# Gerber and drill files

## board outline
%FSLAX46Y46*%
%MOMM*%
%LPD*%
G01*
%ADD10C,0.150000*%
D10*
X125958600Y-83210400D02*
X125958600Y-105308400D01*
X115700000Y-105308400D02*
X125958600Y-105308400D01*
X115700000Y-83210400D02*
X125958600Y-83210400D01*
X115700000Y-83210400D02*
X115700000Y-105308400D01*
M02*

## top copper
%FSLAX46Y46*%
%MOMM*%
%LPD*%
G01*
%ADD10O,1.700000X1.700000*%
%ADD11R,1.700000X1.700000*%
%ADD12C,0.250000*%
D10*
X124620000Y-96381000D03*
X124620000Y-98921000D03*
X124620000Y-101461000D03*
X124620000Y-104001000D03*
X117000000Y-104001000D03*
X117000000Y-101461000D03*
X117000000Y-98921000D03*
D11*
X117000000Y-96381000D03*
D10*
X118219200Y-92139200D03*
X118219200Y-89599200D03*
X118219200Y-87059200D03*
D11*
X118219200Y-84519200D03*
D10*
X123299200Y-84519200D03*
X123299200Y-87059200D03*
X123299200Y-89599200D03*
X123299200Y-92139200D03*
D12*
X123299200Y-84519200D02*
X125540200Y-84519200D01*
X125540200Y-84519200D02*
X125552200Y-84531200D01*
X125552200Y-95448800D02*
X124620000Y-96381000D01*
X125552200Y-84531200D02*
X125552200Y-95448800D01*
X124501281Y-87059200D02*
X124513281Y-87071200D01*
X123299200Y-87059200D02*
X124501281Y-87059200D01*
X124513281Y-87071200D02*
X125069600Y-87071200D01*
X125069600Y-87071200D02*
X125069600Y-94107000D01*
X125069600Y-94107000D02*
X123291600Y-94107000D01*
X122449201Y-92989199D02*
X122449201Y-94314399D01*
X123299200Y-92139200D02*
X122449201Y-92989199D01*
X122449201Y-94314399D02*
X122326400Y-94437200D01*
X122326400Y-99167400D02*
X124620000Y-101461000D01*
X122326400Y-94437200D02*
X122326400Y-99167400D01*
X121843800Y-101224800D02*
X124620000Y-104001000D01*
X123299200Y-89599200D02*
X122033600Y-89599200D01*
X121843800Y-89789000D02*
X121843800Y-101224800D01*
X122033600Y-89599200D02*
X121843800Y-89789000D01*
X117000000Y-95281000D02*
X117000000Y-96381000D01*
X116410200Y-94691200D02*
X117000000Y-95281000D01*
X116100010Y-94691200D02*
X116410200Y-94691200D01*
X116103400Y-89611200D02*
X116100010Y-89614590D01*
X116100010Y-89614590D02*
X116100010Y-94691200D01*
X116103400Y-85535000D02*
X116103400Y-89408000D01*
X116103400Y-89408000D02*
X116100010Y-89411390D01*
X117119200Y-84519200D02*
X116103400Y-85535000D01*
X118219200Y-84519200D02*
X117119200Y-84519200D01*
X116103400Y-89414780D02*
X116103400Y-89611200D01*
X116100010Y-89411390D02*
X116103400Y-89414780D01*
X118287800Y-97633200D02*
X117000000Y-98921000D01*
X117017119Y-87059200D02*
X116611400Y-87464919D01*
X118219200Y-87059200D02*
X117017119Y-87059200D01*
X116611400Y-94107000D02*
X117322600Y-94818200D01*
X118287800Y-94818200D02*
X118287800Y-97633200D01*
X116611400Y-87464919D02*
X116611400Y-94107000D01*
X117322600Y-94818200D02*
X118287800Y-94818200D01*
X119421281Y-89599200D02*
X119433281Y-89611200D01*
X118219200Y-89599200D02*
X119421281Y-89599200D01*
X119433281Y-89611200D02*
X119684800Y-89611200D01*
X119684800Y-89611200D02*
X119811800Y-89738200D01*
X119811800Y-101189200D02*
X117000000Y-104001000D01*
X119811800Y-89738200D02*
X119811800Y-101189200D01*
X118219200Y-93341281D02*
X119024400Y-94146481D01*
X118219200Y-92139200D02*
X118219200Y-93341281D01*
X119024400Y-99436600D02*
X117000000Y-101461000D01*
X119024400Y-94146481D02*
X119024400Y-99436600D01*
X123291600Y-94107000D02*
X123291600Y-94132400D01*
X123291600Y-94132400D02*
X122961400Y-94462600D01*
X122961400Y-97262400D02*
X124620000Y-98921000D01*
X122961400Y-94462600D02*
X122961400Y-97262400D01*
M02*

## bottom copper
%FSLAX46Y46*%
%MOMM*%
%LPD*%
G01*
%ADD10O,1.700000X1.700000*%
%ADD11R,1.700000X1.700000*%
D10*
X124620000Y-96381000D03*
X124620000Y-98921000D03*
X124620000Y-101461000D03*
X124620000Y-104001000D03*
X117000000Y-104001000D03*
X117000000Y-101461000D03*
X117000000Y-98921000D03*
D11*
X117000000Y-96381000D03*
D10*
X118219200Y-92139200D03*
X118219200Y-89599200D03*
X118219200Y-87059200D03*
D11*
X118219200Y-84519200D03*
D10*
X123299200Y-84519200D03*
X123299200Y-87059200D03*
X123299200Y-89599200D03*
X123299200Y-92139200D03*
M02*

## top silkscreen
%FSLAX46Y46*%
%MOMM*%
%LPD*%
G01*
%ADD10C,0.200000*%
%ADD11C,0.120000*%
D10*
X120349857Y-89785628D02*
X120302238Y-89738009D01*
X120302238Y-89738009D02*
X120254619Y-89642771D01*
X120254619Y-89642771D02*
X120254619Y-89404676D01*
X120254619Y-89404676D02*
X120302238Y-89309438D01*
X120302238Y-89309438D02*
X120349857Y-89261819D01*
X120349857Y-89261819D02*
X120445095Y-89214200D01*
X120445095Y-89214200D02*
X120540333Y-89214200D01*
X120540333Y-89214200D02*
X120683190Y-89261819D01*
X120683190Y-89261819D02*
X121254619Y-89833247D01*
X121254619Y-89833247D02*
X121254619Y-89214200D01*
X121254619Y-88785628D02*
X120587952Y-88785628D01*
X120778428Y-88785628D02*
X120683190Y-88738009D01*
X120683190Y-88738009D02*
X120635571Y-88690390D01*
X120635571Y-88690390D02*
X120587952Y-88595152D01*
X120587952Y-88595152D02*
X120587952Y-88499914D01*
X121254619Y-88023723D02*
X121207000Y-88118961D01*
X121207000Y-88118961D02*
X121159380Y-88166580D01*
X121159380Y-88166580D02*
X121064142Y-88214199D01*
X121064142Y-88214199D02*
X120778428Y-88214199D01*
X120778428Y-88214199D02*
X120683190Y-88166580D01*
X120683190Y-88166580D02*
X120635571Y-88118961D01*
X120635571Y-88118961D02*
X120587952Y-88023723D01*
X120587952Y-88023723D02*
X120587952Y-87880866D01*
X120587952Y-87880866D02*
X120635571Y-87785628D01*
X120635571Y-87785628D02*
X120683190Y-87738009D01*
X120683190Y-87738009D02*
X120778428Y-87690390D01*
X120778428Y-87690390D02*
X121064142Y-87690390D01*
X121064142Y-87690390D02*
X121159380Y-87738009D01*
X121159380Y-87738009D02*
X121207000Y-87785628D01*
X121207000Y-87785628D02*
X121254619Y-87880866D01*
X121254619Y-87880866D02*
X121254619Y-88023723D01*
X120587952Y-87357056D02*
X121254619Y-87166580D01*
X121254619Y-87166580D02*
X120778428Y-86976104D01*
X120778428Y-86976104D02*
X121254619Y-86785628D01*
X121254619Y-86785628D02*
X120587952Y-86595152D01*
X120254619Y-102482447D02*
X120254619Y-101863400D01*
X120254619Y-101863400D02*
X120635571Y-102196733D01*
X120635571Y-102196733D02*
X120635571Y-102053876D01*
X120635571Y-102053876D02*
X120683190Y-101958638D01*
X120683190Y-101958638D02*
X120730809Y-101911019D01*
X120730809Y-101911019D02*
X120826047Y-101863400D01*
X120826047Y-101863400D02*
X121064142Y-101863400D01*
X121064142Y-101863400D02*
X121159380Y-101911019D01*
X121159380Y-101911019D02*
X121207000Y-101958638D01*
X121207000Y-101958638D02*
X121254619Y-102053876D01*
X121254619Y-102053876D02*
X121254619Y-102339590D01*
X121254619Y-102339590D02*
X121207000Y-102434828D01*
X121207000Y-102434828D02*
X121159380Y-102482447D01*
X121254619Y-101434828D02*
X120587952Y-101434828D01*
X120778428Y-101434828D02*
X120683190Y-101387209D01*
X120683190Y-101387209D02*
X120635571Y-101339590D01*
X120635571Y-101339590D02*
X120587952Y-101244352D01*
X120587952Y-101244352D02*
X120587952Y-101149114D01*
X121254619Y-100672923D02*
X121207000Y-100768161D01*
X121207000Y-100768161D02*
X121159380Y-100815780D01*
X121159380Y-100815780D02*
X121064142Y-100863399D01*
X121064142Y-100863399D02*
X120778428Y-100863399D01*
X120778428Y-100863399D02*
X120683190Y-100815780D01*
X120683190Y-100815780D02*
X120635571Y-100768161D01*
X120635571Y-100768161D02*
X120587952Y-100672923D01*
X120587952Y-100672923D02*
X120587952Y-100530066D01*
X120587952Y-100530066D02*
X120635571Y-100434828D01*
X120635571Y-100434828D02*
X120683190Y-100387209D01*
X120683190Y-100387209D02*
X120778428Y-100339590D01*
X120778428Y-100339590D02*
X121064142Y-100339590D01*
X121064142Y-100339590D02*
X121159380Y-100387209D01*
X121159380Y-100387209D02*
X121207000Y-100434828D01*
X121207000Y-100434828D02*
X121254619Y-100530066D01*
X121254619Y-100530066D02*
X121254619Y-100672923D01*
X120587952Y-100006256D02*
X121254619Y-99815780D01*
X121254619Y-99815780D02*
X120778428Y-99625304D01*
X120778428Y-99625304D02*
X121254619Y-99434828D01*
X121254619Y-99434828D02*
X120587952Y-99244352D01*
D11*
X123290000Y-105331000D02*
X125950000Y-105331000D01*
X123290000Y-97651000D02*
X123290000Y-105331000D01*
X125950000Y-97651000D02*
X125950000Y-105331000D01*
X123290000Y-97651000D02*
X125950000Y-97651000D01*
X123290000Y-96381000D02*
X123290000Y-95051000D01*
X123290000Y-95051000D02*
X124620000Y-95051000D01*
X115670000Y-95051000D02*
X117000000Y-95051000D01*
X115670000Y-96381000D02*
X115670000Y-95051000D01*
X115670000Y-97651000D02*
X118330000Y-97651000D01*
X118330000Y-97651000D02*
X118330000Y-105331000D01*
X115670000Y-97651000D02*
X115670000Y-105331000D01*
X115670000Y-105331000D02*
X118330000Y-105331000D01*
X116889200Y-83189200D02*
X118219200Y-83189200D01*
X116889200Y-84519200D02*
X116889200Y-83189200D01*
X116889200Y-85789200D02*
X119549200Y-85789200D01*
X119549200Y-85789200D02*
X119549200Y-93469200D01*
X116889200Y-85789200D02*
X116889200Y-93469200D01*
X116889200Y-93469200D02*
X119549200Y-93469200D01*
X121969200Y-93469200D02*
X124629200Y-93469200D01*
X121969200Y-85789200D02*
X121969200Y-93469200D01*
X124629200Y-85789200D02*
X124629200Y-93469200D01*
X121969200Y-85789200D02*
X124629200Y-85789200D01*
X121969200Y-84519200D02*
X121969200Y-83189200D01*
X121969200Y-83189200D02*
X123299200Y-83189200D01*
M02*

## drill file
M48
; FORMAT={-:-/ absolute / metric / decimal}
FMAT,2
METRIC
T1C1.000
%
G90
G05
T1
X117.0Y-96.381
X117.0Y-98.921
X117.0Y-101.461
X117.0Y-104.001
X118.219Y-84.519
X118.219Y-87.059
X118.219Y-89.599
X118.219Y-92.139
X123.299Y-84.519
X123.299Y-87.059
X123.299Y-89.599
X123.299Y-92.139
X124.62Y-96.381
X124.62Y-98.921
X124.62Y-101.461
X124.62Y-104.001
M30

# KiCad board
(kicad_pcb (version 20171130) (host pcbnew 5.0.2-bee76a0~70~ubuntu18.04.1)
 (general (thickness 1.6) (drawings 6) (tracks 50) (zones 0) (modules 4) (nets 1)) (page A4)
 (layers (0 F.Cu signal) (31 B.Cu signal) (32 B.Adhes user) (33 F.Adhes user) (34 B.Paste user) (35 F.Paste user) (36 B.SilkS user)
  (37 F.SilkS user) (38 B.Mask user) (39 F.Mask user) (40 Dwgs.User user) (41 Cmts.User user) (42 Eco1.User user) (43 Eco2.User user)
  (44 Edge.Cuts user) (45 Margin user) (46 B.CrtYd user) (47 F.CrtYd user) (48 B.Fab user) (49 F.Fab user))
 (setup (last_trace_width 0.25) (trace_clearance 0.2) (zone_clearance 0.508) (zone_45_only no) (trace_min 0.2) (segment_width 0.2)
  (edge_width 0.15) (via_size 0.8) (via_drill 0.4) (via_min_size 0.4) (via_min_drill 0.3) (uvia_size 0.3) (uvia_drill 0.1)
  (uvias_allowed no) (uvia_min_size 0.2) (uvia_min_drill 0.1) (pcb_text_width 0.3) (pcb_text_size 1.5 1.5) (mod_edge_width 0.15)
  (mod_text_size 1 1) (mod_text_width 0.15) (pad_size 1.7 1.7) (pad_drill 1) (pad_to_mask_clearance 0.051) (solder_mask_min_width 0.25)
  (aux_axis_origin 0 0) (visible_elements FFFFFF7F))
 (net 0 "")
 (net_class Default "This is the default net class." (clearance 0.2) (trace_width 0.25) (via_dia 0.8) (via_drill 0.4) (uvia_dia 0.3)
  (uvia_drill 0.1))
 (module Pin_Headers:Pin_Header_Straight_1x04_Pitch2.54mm (layer F.Cu) (at 124.62 96.381)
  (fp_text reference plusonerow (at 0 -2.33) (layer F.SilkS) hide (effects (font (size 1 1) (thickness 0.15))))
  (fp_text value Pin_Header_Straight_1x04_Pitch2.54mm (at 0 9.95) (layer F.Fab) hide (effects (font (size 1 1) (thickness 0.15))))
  (fp_line (start -1.33 8.95) (end 1.33 8.95) (layer F.SilkS) (width 0.12))
  (fp_line (start -1.33 1.27) (end -1.33 8.95) (layer F.SilkS) (width 0.12))
  (fp_line (start 1.33 1.27) (end 1.33 8.95) (layer F.SilkS) (width 0.12))
  (fp_line (start -1.33 1.27) (end 1.33 1.27) (layer F.SilkS) (width 0.12))
  (fp_line (start -1.33 0) (end -1.33 -1.33) (layer F.SilkS) (width 0.12))
  (fp_line (start -1.33 -1.33) (end 0 -1.33) (layer F.SilkS) (width 0.12))
  (pad 1 thru_hole oval (at 0 0) (size 1.7 1.7) (drill 1) (layers *.Cu *.Mask))
  (pad 2 thru_hole oval (at 0 2.54) (size 1.7 1.7) (drill 1) (layers *.Cu *.Mask))
  (pad 3 thru_hole oval (at 0 5.08) (size 1.7 1.7) (drill 1) (layers *.Cu *.Mask))
  (pad 4 thru_hole oval (at 0 7.62) (size 1.7 1.7) (drill 1) (layers *.Cu *.Mask)))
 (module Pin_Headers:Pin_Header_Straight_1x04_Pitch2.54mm (layer F.Cu) (at 117 96.381)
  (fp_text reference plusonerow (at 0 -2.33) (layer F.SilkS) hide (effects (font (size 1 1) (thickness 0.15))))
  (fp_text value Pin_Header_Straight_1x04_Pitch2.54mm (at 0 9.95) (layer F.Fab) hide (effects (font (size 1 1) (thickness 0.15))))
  (fp_line (start -1.33 -1.33) (end 0 -1.33) (layer F.SilkS) (width 0.12))
  (fp_line (start -1.33 0) (end -1.33 -1.33) (layer F.SilkS) (width 0.12))
  (fp_line (start -1.33 1.27) (end 1.33 1.27) (layer F.SilkS) (width 0.12))
  (fp_line (start 1.33 1.27) (end 1.33 8.95) (layer F.SilkS) (width 0.12))
  (fp_line (start -1.33 1.27) (end -1.33 8.95) (layer F.SilkS) (width 0.12))
  (fp_line (start -1.33 8.95) (end 1.33 8.95) (layer F.SilkS) (width 0.12))
  (pad 4 thru_hole oval (at 0 7.62) (size 1.7 1.7) (drill 1) (layers *.Cu *.Mask))
  (pad 3 thru_hole oval (at 0 5.08) (size 1.7 1.7) (drill 1) (layers *.Cu *.Mask))
  (pad 2 thru_hole oval (at 0 2.54) (size 1.7 1.7) (drill 1) (layers *.Cu *.Mask))
  (pad 1 thru_hole rect (at 0 0) (size 1.7 1.7) (drill 1) (layers *.Cu *.Mask)))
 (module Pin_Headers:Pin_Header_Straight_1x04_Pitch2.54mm (layer F.Cu) (at 118.2192 84.5192)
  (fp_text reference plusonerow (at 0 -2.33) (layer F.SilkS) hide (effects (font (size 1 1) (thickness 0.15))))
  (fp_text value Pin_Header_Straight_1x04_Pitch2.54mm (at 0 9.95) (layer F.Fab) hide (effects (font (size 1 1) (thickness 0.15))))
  (fp_line (start -1.33 -1.33) (end 0 -1.33) (layer F.SilkS) (width 0.12))
  (fp_line (start -1.33 0) (end -1.33 -1.33) (layer F.SilkS) (width 0.12))
  (fp_line (start -1.33 1.27) (end 1.33 1.27) (layer F.SilkS) (width 0.12))
  (fp_line (start 1.33 1.27) (end 1.33 8.95) (layer F.SilkS) (width 0.12))
  (fp_line (start -1.33 1.27) (end -1.33 8.95) (layer F.SilkS) (width 0.12))
  (fp_line (start -1.33 8.95) (end 1.33 8.95) (layer F.SilkS) (width 0.12))
  (pad 4 thru_hole oval (at 0 7.62) (size 1.7 1.7) (drill 1) (layers *.Cu *.Mask))
  (pad 3 thru_hole oval (at 0 5.08) (size 1.7 1.7) (drill 1) (layers *.Cu *.Mask))
  (pad 2 thru_hole oval (at 0 2.54) (size 1.7 1.7) (drill 1) (layers *.Cu *.Mask))
  (pad 1 thru_hole rect (at 0 0) (size 1.7 1.7) (drill 1) (layers *.Cu *.Mask)))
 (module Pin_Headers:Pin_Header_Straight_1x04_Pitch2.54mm (layer F.Cu) (at 123.2992 84.5192)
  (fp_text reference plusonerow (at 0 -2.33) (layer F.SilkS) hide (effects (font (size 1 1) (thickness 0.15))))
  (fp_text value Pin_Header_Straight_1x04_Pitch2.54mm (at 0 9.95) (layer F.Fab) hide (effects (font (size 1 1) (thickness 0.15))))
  (fp_line (start -1.33 8.95) (end 1.33 8.95) (layer F.SilkS) (width 0.12))
  (fp_line (start -1.33 1.27) (end -1.33 8.95) (layer F.SilkS) (width 0.12))
  (fp_line (start 1.33 1.27) (end 1.33 8.95) (layer F.SilkS) (width 0.12))
  (fp_line (start -1.33 1.27) (end 1.33 1.27) (layer F.SilkS) (width 0.12))
  (fp_line (start -1.33 0) (end -1.33 -1.33) (layer F.SilkS) (width 0.12))
  (fp_line (start -1.33 -1.33) (end 0 -1.33) (layer F.SilkS) (width 0.12))
  (pad 8 thru_hole oval (at 0 0) (size 1.7 1.7) (drill 1) (layers *.Cu *.Mask))
  (pad 7 thru_hole oval (at 0 2.54) (size 1.7 1.7) (drill 1) (layers *.Cu *.Mask))
  (pad 6 thru_hole oval (at 0 5.08) (size 1.7 1.7) (drill 1) (layers *.Cu *.Mask))
  (pad 5 thru_hole oval (at 0 7.62) (size 1.7 1.7) (drill 1) (layers *.Cu *.Mask)))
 (gr_line (start 125.9586 83.2104) (end 125.9586 105.3084) (layer Edge.Cuts) (width 0.15))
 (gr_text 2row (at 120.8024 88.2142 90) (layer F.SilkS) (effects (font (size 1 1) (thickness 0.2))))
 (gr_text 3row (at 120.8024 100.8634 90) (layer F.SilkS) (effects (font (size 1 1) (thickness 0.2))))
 (gr_line (start 115.7 105.3084) (end 125.9586 105.3084) (layer Edge.Cuts) (width 0.15))
 (gr_line (start 115.7 83.2104) (end 125.9586 83.2104) (layer Edge.Cuts) (width 0.15))
 (gr_line (start 115.7 83.2104) (end 115.7 105.3084) (layer Edge.Cuts) (width 0.15))
 (segment (start 123.2992 84.5192) (end 125.5402 84.5192) (width 0.25) (layer F.Cu) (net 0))
 (segment (start 125.5402 84.5192) (end 125.5522 84.5312) (width 0.25) (layer F.Cu) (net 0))
 (segment (start 125.5522 95.4488) (end 124.62 96.381) (width 0.25) (layer F.Cu) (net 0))
 (segment (start 125.5522 84.5312) (end 125.5522 95.4488) (width 0.25) (layer F.Cu) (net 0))
 (segment (start 124.501281 87.0592) (end 124.513281 87.0712) (width 0.25) (layer F.Cu) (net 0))
 (segment (start 123.2992 87.0592) (end 124.501281 87.0592) (width 0.25) (layer F.Cu) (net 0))
 (segment (start 124.513281 87.0712) (end 125.0696 87.0712) (width 0.25) (layer F.Cu) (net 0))
 (segment (start 125.0696 87.0712) (end 125.0696 94.107) (width 0.25) (layer F.Cu) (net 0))
 (segment (start 125.0696 94.107) (end 123.2916 94.107) (width 0.25) (layer F.Cu) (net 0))
 (segment (start 122.449201 92.989199) (end 122.449201 94.314399) (width 0.25) (layer F.Cu) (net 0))
 (segment (start 123.2992 92.1392) (end 122.449201 92.989199) (width 0.25) (layer F.Cu) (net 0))
 (segment (start 122.449201 94.314399) (end 122.3264 94.4372) (width 0.25) (layer F.Cu) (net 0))
 (segment (start 122.3264 99.1674) (end 124.62 101.461) (width 0.25) (layer F.Cu) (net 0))
 (segment (start 122.3264 94.4372) (end 122.3264 99.1674) (width 0.25) (layer F.Cu) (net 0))
 (segment (start 121.8438 101.2248) (end 124.62 104.001) (width 0.25) (layer F.Cu) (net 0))
 (segment (start 123.2992 89.5992) (end 122.0336 89.5992) (width 0.25) (layer F.Cu) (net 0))
 (segment (start 121.8438 89.789) (end 121.8438 101.2248) (width 0.25) (layer F.Cu) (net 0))
 (segment (start 122.0336 89.5992) (end 121.8438 89.789) (width 0.25) (layer F.Cu) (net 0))
 (segment (start 117 95.281) (end 117 96.381) (width 0.25) (layer F.Cu) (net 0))
 (segment (start 116.4102 94.6912) (end 117 95.281) (width 0.25) (layer F.Cu) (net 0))
 (segment (start 116.10001 94.6912) (end 116.4102 94.6912) (width 0.25) (layer F.Cu) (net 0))
 (segment (start 116.1034 89.6112) (end 116.10001 89.61459) (width 0.25) (layer F.Cu) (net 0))
 (segment (start 116.10001 89.61459) (end 116.10001 94.6912) (width 0.25) (layer F.Cu) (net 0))
 (segment (start 116.1034 85.535) (end 116.1034 89.408) (width 0.25) (layer F.Cu) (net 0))
 (segment (start 116.1034 89.408) (end 116.10001 89.41139) (width 0.25) (layer F.Cu) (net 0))
 (segment (start 117.1192 84.5192) (end 116.1034 85.535) (width 0.25) (layer F.Cu) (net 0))
 (segment (start 118.2192 84.5192) (end 117.1192 84.5192) (width 0.25) (layer F.Cu) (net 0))
 (segment (start 116.1034 89.41478) (end 116.1034 89.6112) (width 0.25) (layer F.Cu) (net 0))
 (segment (start 116.10001 89.41139) (end 116.1034 89.41478) (width 0.25) (layer F.Cu) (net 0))
 (segment (start 118.2878 97.6332) (end 117 98.921) (width 0.25) (layer F.Cu) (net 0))
 (segment (start 117.017119 87.0592) (end 116.6114 87.464919) (width 0.25) (layer F.Cu) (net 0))
 (segment (start 118.2192 87.0592) (end 117.017119 87.0592) (width 0.25) (layer F.Cu) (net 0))
 (segment (start 116.6114 94.107) (end 117.3226 94.8182) (width 0.25) (layer F.Cu) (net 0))
 (segment (start 118.2878 94.8182) (end 118.2878 97.6332) (width 0.25) (layer F.Cu) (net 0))
 (segment (start 116.6114 87.464919) (end 116.6114 94.107) (width 0.25) (layer F.Cu) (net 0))
 (segment (start 117.3226 94.8182) (end 118.2878 94.8182) (width 0.25) (layer F.Cu) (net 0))
 (segment (start 119.421281 89.5992) (end 119.433281 89.6112) (width 0.25) (layer F.Cu) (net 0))
 (segment (start 118.2192 89.5992) (end 119.421281 89.5992) (width 0.25) (layer F.Cu) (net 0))
 (segment (start 119.433281 89.6112) (end 119.6848 89.6112) (width 0.25) (layer F.Cu) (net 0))
 (segment (start 119.6848 89.6112) (end 119.8118 89.7382) (width 0.25) (layer F.Cu) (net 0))
 (segment (start 119.8118 101.1892) (end 117 104.001) (width 0.25) (layer F.Cu) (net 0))
 (segment (start 119.8118 89.7382) (end 119.8118 101.1892) (width 0.25) (layer F.Cu) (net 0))
 (segment (start 118.2192 93.341281) (end 119.0244 94.146481) (width 0.25) (layer F.Cu) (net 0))
 (segment (start 118.2192 92.1392) (end 118.2192 93.341281) (width 0.25) (layer F.Cu) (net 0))
 (segment (start 119.0244 99.4366) (end 117 101.461) (width 0.25) (layer F.Cu) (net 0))
 (segment (start 119.0244 94.146481) (end 119.0244 99.4366) (width 0.25) (layer F.Cu) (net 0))
 (segment (start 123.2916 94.107) (end 123.2916 94.1324) (width 0.25) (layer F.Cu) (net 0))
 (segment (start 123.2916 94.1324) (end 122.9614 94.4626) (width 0.25) (layer F.Cu) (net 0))
 (segment (start 122.9614 97.2624) (end 124.62 98.921) (width 0.25) (layer F.Cu) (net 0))
 (segment (start 122.9614 94.4626) (end 122.9614 97.2624) (width 0.25) (layer F.Cu) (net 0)))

